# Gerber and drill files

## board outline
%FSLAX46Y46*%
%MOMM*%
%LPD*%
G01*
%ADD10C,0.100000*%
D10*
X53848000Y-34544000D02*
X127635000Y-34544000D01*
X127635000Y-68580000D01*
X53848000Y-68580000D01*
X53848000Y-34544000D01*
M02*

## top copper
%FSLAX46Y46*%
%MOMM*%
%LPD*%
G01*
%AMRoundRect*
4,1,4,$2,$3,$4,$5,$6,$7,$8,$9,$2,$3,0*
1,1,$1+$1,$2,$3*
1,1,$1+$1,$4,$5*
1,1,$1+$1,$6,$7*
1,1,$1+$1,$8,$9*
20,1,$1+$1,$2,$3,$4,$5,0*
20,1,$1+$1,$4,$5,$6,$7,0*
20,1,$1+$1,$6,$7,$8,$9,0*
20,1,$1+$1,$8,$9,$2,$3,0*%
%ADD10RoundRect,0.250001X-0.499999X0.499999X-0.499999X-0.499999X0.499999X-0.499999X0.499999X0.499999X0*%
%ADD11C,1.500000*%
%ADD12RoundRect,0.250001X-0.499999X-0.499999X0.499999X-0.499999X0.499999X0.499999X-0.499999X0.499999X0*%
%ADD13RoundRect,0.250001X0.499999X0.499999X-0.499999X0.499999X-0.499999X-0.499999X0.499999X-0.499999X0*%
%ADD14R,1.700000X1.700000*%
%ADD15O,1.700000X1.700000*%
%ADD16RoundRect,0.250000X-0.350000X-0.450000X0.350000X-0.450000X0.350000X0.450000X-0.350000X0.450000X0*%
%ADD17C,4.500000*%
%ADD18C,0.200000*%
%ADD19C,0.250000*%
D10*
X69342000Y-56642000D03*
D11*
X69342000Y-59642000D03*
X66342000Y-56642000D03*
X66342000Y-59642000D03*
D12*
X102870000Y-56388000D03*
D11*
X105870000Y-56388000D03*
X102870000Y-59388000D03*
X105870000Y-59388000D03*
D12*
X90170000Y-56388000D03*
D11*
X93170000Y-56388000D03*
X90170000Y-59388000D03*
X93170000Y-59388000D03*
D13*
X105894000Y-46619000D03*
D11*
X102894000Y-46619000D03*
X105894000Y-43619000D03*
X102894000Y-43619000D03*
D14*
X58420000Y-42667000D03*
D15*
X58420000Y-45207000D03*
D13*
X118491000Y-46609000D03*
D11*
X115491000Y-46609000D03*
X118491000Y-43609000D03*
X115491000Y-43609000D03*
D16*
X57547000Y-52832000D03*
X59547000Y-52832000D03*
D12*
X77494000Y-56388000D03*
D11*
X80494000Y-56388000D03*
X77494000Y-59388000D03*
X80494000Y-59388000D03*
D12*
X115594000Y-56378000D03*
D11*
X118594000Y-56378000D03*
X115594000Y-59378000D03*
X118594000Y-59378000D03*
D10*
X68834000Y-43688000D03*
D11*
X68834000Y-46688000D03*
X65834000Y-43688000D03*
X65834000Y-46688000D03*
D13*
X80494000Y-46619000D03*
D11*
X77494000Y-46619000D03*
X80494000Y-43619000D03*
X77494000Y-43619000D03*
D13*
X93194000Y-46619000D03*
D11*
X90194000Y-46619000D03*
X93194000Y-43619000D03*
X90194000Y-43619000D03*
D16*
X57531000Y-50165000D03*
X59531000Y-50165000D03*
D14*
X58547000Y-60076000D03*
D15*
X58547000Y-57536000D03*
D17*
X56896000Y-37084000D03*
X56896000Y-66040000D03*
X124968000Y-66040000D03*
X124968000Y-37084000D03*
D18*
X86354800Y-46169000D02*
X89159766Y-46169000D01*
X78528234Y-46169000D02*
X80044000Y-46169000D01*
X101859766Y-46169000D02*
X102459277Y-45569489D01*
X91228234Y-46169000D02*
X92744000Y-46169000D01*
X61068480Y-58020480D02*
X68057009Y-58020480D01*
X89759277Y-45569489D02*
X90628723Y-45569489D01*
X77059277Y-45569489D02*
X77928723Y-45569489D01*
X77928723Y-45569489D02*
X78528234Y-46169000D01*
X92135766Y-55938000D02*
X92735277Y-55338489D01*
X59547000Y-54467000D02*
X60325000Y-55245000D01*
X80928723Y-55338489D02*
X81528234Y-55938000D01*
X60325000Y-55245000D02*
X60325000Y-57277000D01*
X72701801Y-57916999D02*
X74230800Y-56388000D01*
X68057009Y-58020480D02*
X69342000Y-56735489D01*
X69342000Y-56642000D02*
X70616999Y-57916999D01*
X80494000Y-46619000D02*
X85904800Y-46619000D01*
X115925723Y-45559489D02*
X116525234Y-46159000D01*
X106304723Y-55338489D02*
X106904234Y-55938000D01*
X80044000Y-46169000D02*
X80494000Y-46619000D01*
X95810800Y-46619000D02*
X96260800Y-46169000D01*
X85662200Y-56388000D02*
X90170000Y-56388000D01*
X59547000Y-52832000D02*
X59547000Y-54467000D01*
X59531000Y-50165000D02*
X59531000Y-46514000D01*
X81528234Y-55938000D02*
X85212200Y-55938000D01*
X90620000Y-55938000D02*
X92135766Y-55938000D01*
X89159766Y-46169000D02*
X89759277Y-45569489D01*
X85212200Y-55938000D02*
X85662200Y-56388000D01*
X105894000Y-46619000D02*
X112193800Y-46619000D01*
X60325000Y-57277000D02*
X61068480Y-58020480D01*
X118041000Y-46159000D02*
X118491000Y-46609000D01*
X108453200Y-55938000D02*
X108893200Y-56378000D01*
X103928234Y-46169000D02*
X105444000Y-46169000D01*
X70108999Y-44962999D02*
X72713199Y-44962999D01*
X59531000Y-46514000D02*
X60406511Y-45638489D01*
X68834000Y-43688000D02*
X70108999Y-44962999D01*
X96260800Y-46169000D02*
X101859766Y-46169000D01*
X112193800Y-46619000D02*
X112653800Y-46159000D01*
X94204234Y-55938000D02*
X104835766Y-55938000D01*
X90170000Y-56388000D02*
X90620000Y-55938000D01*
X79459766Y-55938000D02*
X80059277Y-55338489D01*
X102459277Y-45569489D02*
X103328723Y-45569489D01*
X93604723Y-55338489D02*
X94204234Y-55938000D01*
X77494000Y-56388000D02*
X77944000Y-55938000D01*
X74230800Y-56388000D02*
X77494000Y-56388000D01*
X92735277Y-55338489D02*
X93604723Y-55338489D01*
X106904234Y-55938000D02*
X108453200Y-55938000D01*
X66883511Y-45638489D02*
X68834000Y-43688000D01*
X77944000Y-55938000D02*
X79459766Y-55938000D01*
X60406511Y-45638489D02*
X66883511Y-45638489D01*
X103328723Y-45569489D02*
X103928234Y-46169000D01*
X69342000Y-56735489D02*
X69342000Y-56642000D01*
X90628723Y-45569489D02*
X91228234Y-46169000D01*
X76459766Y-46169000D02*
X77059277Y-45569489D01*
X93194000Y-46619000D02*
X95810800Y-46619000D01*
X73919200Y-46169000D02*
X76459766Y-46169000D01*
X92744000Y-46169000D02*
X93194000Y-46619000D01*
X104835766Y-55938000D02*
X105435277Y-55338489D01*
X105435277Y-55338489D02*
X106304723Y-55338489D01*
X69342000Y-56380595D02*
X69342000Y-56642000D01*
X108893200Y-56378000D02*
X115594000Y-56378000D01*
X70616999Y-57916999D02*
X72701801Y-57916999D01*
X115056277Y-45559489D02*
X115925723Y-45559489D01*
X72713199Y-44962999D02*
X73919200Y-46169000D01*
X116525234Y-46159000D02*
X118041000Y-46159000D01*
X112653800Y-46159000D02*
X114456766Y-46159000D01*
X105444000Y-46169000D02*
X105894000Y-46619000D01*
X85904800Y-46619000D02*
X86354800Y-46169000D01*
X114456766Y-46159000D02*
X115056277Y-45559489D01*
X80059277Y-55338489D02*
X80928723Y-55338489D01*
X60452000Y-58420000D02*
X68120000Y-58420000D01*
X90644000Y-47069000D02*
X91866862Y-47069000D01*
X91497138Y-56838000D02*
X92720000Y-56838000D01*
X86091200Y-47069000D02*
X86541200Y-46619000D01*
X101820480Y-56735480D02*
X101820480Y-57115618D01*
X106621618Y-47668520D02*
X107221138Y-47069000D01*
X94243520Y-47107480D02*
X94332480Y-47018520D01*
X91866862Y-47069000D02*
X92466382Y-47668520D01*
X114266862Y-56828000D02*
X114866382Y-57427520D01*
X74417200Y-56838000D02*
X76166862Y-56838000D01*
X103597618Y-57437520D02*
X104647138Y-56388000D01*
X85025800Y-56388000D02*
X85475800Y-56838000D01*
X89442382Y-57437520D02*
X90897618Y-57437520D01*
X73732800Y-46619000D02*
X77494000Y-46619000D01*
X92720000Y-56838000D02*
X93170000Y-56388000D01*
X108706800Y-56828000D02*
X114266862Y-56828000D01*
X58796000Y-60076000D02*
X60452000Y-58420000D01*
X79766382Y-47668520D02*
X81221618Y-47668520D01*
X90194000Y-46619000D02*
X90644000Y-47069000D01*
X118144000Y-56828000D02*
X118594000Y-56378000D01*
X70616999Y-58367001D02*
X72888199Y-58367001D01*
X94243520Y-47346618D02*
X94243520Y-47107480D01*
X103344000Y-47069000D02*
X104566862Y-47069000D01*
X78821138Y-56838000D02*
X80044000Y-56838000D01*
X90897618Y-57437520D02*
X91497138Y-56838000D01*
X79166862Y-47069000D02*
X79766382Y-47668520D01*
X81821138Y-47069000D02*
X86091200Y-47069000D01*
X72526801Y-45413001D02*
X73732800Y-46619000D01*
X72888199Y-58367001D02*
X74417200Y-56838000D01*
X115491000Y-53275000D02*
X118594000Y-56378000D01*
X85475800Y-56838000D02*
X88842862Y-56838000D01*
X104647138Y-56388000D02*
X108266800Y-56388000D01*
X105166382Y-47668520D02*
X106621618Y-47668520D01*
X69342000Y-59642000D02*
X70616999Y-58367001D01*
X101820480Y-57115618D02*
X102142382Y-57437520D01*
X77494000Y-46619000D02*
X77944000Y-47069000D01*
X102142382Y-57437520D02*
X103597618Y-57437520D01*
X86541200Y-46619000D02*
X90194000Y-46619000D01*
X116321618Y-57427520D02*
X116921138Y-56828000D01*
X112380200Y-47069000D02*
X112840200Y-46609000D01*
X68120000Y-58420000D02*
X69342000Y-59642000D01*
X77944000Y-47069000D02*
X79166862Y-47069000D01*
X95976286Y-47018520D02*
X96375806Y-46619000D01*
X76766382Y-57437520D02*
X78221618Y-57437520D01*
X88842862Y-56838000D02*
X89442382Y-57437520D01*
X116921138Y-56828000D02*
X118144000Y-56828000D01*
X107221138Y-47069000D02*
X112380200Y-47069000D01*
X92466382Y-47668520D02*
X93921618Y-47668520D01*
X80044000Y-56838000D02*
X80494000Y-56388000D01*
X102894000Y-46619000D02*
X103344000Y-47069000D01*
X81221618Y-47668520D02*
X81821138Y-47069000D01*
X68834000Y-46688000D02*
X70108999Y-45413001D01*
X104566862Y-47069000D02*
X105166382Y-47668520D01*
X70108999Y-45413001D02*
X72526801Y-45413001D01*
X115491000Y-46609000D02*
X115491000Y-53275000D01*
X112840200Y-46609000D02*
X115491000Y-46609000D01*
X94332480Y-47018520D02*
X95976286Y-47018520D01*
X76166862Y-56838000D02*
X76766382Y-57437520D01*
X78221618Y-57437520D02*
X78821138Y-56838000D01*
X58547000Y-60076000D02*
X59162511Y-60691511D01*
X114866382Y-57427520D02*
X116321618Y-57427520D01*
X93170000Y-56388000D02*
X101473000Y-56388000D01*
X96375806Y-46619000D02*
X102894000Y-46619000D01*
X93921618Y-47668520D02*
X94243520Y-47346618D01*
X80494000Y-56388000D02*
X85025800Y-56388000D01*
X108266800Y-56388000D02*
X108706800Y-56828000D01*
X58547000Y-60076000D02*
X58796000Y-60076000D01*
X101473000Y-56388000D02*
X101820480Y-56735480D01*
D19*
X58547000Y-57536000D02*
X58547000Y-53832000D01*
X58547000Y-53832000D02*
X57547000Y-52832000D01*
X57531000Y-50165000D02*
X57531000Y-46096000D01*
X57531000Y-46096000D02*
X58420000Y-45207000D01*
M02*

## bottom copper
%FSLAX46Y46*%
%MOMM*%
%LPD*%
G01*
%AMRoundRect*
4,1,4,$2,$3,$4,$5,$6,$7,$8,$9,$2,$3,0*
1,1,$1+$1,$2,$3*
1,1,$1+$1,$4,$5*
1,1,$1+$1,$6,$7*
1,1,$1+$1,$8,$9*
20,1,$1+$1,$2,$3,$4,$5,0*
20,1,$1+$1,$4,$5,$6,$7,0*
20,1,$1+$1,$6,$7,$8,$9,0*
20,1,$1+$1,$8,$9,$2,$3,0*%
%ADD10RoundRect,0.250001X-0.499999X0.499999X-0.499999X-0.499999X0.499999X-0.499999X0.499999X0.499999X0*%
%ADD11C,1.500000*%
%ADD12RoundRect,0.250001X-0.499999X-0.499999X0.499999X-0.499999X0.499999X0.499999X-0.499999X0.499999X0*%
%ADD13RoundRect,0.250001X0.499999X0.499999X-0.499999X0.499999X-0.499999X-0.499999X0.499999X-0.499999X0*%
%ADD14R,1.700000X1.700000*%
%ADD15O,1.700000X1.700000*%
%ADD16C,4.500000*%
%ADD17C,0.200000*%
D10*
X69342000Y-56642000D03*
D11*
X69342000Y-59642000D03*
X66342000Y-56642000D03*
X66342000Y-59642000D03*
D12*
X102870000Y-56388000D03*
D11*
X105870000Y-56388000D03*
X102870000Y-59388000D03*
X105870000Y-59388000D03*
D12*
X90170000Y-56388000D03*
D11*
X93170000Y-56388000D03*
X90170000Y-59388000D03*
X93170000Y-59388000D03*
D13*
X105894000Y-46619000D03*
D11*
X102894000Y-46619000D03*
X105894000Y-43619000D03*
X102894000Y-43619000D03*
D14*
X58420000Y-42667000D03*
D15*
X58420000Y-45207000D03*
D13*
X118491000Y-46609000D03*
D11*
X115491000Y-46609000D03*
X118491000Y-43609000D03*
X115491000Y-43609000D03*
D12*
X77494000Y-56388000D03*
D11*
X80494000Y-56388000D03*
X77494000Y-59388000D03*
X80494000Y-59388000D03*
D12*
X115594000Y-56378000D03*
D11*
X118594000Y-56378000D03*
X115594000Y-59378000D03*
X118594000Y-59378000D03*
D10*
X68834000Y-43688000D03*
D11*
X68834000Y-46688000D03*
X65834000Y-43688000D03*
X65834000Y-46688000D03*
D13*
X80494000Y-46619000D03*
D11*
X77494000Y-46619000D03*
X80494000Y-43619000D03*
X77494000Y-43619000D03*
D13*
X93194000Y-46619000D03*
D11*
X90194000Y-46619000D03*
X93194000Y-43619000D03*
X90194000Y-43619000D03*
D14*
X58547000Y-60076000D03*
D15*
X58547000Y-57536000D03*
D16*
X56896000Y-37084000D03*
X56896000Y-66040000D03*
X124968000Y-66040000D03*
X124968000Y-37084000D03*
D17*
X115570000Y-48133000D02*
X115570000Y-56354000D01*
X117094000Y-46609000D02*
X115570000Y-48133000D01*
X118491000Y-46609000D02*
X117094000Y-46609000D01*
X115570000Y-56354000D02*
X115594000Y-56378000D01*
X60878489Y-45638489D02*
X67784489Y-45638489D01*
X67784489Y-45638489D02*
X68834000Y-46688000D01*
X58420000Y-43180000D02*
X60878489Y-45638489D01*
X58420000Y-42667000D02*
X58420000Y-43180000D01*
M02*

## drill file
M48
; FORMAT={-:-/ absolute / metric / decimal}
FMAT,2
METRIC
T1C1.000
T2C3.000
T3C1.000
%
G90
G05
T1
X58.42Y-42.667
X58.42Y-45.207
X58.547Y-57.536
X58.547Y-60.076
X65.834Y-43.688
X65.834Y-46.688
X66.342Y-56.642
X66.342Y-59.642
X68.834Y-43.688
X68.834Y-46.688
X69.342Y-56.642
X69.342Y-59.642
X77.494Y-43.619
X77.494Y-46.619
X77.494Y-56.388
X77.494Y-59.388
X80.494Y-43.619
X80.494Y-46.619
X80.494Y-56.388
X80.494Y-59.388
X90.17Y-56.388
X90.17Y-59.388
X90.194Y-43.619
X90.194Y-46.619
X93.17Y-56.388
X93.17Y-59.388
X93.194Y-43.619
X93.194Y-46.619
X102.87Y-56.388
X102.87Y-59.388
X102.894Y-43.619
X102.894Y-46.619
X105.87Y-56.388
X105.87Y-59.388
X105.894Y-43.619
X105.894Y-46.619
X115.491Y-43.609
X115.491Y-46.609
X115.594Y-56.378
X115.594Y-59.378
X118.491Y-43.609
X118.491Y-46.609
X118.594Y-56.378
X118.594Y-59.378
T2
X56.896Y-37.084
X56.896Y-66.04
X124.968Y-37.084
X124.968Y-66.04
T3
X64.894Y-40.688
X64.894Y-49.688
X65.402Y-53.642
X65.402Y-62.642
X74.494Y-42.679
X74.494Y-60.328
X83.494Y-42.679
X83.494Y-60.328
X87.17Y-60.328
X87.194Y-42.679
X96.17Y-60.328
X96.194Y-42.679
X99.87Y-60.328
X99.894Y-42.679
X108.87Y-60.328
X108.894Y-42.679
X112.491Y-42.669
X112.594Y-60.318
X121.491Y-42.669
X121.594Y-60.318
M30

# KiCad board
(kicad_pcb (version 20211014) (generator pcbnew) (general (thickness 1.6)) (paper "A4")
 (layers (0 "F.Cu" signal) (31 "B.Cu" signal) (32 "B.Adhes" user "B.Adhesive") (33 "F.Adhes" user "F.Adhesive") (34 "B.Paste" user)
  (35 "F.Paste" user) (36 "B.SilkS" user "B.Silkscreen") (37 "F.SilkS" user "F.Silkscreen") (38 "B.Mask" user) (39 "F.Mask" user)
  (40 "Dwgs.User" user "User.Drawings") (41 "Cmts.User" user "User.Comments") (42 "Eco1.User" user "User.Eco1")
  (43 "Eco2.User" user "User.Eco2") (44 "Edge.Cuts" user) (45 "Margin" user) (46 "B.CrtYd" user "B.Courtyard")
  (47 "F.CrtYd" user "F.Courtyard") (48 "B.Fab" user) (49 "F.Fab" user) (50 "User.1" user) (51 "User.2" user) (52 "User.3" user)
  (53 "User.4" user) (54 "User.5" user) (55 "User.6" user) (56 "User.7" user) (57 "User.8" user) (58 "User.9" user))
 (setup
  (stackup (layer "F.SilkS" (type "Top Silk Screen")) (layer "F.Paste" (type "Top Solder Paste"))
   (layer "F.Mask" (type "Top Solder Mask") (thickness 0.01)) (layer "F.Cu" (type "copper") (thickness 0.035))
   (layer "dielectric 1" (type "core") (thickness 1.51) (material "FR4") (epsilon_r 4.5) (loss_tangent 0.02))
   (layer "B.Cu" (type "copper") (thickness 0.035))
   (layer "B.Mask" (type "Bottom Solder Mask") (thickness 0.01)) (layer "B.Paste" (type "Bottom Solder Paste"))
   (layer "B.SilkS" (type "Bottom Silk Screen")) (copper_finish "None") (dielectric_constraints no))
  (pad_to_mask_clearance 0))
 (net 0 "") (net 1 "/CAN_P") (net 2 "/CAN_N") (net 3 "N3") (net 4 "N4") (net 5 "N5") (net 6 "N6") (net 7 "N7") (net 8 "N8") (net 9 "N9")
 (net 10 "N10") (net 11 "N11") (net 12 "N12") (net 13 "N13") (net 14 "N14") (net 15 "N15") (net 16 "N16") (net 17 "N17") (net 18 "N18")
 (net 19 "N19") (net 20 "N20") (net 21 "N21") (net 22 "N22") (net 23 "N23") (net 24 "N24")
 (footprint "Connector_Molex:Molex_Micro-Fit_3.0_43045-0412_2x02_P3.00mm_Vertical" (layer "F.Cu") (at 69.342 56.642 -90)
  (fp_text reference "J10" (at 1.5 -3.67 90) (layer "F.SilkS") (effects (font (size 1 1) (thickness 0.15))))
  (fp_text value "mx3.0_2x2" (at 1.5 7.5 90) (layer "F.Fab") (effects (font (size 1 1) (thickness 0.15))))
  (pad "" np_thru_hole circle locked (at -3 3.94 270) (size 1 1) (drill 1) (layers *.Cu *.Mask))
  (pad "" np_thru_hole circle locked (at 6 3.94 270) (size 1 1) (drill 1) (layers *.Cu *.Mask))
  (pad "1" thru_hole roundrect locked (at 0 0 270) (size 1.5 1.5) (drill 1) (layers *.Cu *.Mask) (roundrect_rratio 0.166667)
   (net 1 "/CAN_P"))
  (pad "2" thru_hole circle locked (at 3 0 270) (size 1.5 1.5) (drill 1) (layers *.Cu *.Mask) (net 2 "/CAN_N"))
  (pad "3" thru_hole circle locked (at 0 3 270) (size 1.5 1.5) (drill 1) (layers *.Cu *.Mask) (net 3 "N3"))
  (pad "4" thru_hole circle locked (at 3 3 270) (size 1.5 1.5) (drill 1) (layers *.Cu *.Mask) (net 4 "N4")))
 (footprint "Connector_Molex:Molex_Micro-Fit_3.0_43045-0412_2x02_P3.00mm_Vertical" (layer "F.Cu") (at 102.87 56.388)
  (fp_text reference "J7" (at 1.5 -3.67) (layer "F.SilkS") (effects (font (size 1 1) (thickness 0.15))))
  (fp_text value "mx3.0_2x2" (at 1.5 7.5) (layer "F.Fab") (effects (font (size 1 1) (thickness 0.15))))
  (pad "" np_thru_hole circle locked (at 6 3.94) (size 1 1) (drill 1) (layers *.Cu *.Mask))
  (pad "" np_thru_hole circle locked (at -3 3.94) (size 1 1) (drill 1) (layers *.Cu *.Mask))
  (pad "1" thru_hole roundrect locked (at 0 0) (size 1.5 1.5) (drill 1) (layers *.Cu *.Mask) (roundrect_rratio 0.166667) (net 1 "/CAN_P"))
  (pad "2" thru_hole circle locked (at 3 0) (size 1.5 1.5) (drill 1) (layers *.Cu *.Mask) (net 2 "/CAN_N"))
  (pad "3" thru_hole circle locked (at 0 3) (size 1.5 1.5) (drill 1) (layers *.Cu *.Mask) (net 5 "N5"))
  (pad "4" thru_hole circle locked (at 3 3) (size 1.5 1.5) (drill 1) (layers *.Cu *.Mask) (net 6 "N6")))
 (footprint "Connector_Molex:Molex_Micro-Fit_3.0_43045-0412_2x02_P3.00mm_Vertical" (layer "F.Cu") (at 90.17 56.388)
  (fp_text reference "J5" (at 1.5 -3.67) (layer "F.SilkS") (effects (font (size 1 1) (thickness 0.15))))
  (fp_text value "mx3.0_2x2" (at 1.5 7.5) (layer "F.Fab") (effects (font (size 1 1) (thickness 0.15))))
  (pad "" np_thru_hole circle locked (at -3 3.94) (size 1 1) (drill 1) (layers *.Cu *.Mask))
  (pad "" np_thru_hole circle locked (at 6 3.94) (size 1 1) (drill 1) (layers *.Cu *.Mask))
  (pad "1" thru_hole roundrect locked (at 0 0) (size 1.5 1.5) (drill 1) (layers *.Cu *.Mask) (roundrect_rratio 0.166667) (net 1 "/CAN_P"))
  (pad "2" thru_hole circle locked (at 3 0) (size 1.5 1.5) (drill 1) (layers *.Cu *.Mask) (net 2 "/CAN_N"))
  (pad "3" thru_hole circle locked (at 0 3) (size 1.5 1.5) (drill 1) (layers *.Cu *.Mask) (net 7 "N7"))
  (pad "4" thru_hole circle locked (at 3 3) (size 1.5 1.5) (drill 1) (layers *.Cu *.Mask) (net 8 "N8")))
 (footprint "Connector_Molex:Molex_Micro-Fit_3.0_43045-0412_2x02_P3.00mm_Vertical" (layer "F.Cu") (at 105.894 46.619 180)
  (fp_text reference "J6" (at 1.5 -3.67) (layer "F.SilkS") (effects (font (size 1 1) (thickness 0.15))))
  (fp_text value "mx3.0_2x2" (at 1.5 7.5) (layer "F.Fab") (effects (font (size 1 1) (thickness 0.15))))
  (pad "" np_thru_hole circle locked (at 6 3.94 180) (size 1 1) (drill 1) (layers *.Cu *.Mask))
  (pad "" np_thru_hole circle locked (at -3 3.94 180) (size 1 1) (drill 1) (layers *.Cu *.Mask))
  (pad "1" thru_hole roundrect locked (at 0 0 180) (size 1.5 1.5) (drill 1) (layers *.Cu *.Mask) (roundrect_rratio 0.166667)
   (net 1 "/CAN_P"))
  (pad "2" thru_hole circle locked (at 3 0 180) (size 1.5 1.5) (drill 1) (layers *.Cu *.Mask) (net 2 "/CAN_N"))
  (pad "3" thru_hole circle locked (at 0 3 180) (size 1.5 1.5) (drill 1) (layers *.Cu *.Mask) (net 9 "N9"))
  (pad "4" thru_hole circle locked (at 3 3 180) (size 1.5 1.5) (drill 1) (layers *.Cu *.Mask) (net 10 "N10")))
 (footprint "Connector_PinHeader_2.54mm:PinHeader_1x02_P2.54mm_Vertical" (layer "F.Cu") (at 58.42 42.667)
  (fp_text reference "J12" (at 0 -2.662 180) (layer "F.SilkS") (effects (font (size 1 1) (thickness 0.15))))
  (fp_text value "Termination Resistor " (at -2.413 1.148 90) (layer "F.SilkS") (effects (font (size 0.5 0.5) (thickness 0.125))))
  (pad "1" thru_hole rect locked (at 0 0) (size 1.7 1.7) (drill 1) (layers *.Cu *.Mask) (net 2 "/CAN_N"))
  (pad "2" thru_hole oval locked (at 0 2.54) (size 1.7 1.7) (drill 1) (layers *.Cu *.Mask) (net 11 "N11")))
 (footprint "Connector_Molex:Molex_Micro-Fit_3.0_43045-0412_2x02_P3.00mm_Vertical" (layer "F.Cu") (at 118.491 46.609 180)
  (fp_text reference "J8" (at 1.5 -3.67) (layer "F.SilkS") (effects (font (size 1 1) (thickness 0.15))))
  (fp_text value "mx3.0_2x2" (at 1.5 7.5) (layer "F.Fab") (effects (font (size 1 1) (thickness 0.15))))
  (pad "" np_thru_hole circle locked (at 6 3.94 180) (size 1 1) (drill 1) (layers *.Cu *.Mask))
  (pad "" np_thru_hole circle locked (at -3 3.94 180) (size 1 1) (drill 1) (layers *.Cu *.Mask))
  (pad "1" thru_hole roundrect locked (at 0 0 180) (size 1.5 1.5) (drill 1) (layers *.Cu *.Mask) (roundrect_rratio 0.166667)
   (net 1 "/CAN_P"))
  (pad "2" thru_hole circle locked (at 3 0 180) (size 1.5 1.5) (drill 1) (layers *.Cu *.Mask) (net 2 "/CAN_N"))
  (pad "3" thru_hole circle locked (at 0 3 180) (size 1.5 1.5) (drill 1) (layers *.Cu *.Mask) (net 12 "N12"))
  (pad "4" thru_hole circle locked (at 3 3 180) (size 1.5 1.5) (drill 1) (layers *.Cu *.Mask) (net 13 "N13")))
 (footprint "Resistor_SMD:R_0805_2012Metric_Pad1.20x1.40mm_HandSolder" (layer "F.Cu") (at 58.547 52.832)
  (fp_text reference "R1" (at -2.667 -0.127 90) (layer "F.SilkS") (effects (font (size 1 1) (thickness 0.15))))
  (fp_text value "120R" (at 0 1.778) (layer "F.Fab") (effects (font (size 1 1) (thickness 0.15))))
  (pad "1" smd roundrect locked (at -1 0) (size 1.2 1.4) (layers "F.Cu" "F.Paste" "F.Mask") (roundrect_rratio 0.208333) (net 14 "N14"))
  (pad "2" smd roundrect locked (at 1 0) (size 1.2 1.4) (layers "F.Cu" "F.Paste" "F.Mask") (roundrect_rratio 0.208333) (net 1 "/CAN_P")))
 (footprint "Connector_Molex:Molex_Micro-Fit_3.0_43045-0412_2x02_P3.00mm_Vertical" (layer "F.Cu") (at 77.494 56.388)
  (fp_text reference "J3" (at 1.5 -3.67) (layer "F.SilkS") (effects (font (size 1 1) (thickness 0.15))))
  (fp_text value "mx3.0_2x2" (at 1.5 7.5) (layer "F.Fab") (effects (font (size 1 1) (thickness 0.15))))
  (pad "" np_thru_hole circle locked (at -3 3.94) (size 1 1) (drill 1) (layers *.Cu *.Mask))
  (pad "" np_thru_hole circle locked (at 6 3.94) (size 1 1) (drill 1) (layers *.Cu *.Mask))
  (pad "1" thru_hole roundrect locked (at 0 0) (size 1.5 1.5) (drill 1) (layers *.Cu *.Mask) (roundrect_rratio 0.166667) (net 1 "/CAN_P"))
  (pad "2" thru_hole circle locked (at 3 0) (size 1.5 1.5) (drill 1) (layers *.Cu *.Mask) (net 2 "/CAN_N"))
  (pad "3" thru_hole circle locked (at 0 3) (size 1.5 1.5) (drill 1) (layers *.Cu *.Mask) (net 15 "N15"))
  (pad "4" thru_hole circle locked (at 3 3) (size 1.5 1.5) (drill 1) (layers *.Cu *.Mask) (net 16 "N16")))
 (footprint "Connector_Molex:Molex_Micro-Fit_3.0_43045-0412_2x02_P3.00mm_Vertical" (layer "F.Cu") (at 115.594 56.378)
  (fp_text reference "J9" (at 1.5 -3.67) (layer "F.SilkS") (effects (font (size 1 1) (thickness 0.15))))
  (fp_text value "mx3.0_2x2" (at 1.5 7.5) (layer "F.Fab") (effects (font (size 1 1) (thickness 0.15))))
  (pad "" np_thru_hole circle locked (at 6 3.94) (size 1 1) (drill 1) (layers *.Cu *.Mask))
  (pad "" np_thru_hole circle locked (at -3 3.94) (size 1 1) (drill 1) (layers *.Cu *.Mask))
  (pad "1" thru_hole roundrect locked (at 0 0) (size 1.5 1.5) (drill 1) (layers *.Cu *.Mask) (roundrect_rratio 0.166667) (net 1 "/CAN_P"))
  (pad "2" thru_hole circle locked (at 3 0) (size 1.5 1.5) (drill 1) (layers *.Cu *.Mask) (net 2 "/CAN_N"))
  (pad "3" thru_hole circle locked (at 0 3) (size 1.5 1.5) (drill 1) (layers *.Cu *.Mask) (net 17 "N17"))
  (pad "4" thru_hole circle locked (at 3 3) (size 1.5 1.5) (drill 1) (layers *.Cu *.Mask) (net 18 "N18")))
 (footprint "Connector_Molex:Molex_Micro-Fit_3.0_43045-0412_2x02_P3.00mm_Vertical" (layer "F.Cu") (at 68.834 43.688 -90)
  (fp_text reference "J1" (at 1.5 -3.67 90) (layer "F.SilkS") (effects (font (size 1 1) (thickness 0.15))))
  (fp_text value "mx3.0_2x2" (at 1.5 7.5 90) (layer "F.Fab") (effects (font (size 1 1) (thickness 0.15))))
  (pad "" np_thru_hole circle locked (at -3 3.94 270) (size 1 1) (drill 1) (layers *.Cu *.Mask))
  (pad "" np_thru_hole circle locked (at 6 3.94 270) (size 1 1) (drill 1) (layers *.Cu *.Mask))
  (pad "1" thru_hole roundrect locked (at 0 0 270) (size 1.5 1.5) (drill 1) (layers *.Cu *.Mask) (roundrect_rratio 0.166667)
   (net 1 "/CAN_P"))
  (pad "2" thru_hole circle locked (at 3 0 270) (size 1.5 1.5) (drill 1) (layers *.Cu *.Mask) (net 2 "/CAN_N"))
  (pad "3" thru_hole circle locked (at 0 3 270) (size 1.5 1.5) (drill 1) (layers *.Cu *.Mask) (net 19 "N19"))
  (pad "4" thru_hole circle locked (at 3 3 270) (size 1.5 1.5) (drill 1) (layers *.Cu *.Mask) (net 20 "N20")))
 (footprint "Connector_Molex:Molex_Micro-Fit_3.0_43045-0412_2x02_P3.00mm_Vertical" (layer "F.Cu") (at 80.494 46.619 180)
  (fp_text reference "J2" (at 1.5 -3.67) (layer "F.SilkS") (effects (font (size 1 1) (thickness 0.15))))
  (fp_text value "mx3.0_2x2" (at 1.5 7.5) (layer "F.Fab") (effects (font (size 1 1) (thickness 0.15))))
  (pad "" np_thru_hole circle locked (at -3 3.94 180) (size 1 1) (drill 1) (layers *.Cu *.Mask))
  (pad "" np_thru_hole circle locked (at 6 3.94 180) (size 1 1) (drill 1) (layers *.Cu *.Mask))
  (pad "1" thru_hole roundrect locked (at 0 0 180) (size 1.5 1.5) (drill 1) (layers *.Cu *.Mask) (roundrect_rratio 0.166667)
   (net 1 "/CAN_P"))
  (pad "2" thru_hole circle locked (at 3 0 180) (size 1.5 1.5) (drill 1) (layers *.Cu *.Mask) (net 2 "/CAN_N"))
  (pad "3" thru_hole circle locked (at 0 3 180) (size 1.5 1.5) (drill 1) (layers *.Cu *.Mask) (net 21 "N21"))
  (pad "4" thru_hole circle locked (at 3 3 180) (size 1.5 1.5) (drill 1) (layers *.Cu *.Mask) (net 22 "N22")))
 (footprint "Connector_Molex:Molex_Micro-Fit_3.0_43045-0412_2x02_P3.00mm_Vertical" (layer "F.Cu") (at 93.194 46.619 180)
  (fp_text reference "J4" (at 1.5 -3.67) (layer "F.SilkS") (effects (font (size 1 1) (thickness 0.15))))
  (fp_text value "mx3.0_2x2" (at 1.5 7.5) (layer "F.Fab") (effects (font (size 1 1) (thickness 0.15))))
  (pad "" np_thru_hole circle locked (at -3 3.94 180) (size 1 1) (drill 1) (layers *.Cu *.Mask))
  (pad "" np_thru_hole circle locked (at 6 3.94 180) (size 1 1) (drill 1) (layers *.Cu *.Mask))
  (pad "1" thru_hole roundrect locked (at 0 0 180) (size 1.5 1.5) (drill 1) (layers *.Cu *.Mask) (roundrect_rratio 0.166667)
   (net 1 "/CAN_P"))
  (pad "2" thru_hole circle locked (at 3 0 180) (size 1.5 1.5) (drill 1) (layers *.Cu *.Mask) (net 2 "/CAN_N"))
  (pad "3" thru_hole circle locked (at 0 3 180) (size 1.5 1.5) (drill 1) (layers *.Cu *.Mask) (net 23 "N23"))
  (pad "4" thru_hole circle locked (at 3 3 180) (size 1.5 1.5) (drill 1) (layers *.Cu *.Mask) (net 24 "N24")))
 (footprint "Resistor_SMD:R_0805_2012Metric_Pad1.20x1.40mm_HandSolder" (layer "F.Cu") (at 58.531 50.165)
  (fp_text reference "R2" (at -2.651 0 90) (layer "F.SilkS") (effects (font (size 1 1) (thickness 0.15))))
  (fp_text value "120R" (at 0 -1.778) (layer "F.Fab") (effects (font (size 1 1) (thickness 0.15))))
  (pad "1" smd roundrect locked (at -1 0) (size 1.2 1.4) (layers "F.Cu" "F.Paste" "F.Mask") (roundrect_rratio 0.208333) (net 11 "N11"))
  (pad "2" smd roundrect locked (at 1 0) (size 1.2 1.4) (layers "F.Cu" "F.Paste" "F.Mask") (roundrect_rratio 0.208333) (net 1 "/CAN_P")))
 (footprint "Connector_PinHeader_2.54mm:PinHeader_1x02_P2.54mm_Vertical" (layer "F.Cu") (at 58.547 60.076 180)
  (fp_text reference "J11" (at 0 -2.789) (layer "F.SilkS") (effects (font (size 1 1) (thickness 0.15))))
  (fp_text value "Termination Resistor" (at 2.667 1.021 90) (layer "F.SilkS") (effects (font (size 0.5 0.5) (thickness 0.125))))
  (pad "1" thru_hole rect locked (at 0 0 180) (size 1.7 1.7) (drill 1) (layers *.Cu *.Mask) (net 2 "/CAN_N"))
  (pad "2" thru_hole oval locked (at 0 2.54 180) (size 1.7 1.7) (drill 1) (layers *.Cu *.Mask) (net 14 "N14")))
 (gr_rect (start 127.635 34.544) (end 53.848 68.58) (layer "Edge.Cuts") (width 0.1) (fill none))
 (via (at 56.896 37.084) (size 4.5) (drill 3) (layers "F.Cu" "B.Cu") (free) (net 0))
 (via (at 56.896 66.04) (size 4.5) (drill 3) (layers "F.Cu" "B.Cu") (free) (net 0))
 (via (at 124.968 66.04) (size 4.5) (drill 3) (layers "F.Cu" "B.Cu") (free) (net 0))
 (via (at 124.968 37.084) (size 4.5) (drill 3) (layers "F.Cu" "B.Cu") (free) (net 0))
 (segment (start 86.3548 46.169) (end 89.159766 46.169) (width 0.2) (layer "F.Cu") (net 1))
 (segment (start 78.528234 46.169) (end 80.044 46.169) (width 0.2) (layer "F.Cu") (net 1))
 (segment (start 101.859766 46.169) (end 102.459277 45.569489) (width 0.2) (layer "F.Cu") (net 1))
 (segment (start 91.228234 46.169) (end 92.744 46.169) (width 0.2) (layer "F.Cu") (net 1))
 (segment (start 61.06848 58.02048) (end 68.057009 58.02048) (width 0.2) (layer "F.Cu") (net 1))
 (segment (start 89.759277 45.569489) (end 90.628723 45.569489) (width 0.2) (layer "F.Cu") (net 1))
 (segment (start 77.059277 45.569489) (end 77.928723 45.569489) (width 0.2) (layer "F.Cu") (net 1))
 (segment (start 77.928723 45.569489) (end 78.528234 46.169) (width 0.2) (layer "F.Cu") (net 1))
 (segment (start 92.135766 55.938) (end 92.735277 55.338489) (width 0.2) (layer "F.Cu") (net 1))
 (segment (start 59.547 54.467) (end 60.325 55.245) (width 0.2) (layer "F.Cu") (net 1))
 (segment (start 80.928723 55.338489) (end 81.528234 55.938) (width 0.2) (layer "F.Cu") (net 1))
 (segment (start 60.325 55.245) (end 60.325 57.277) (width 0.2) (layer "F.Cu") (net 1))
 (segment (start 72.701801 57.916999) (end 74.2308 56.388) (width 0.2) (layer "F.Cu") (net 1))
 (segment (start 68.057009 58.02048) (end 69.342 56.735489) (width 0.2) (layer "F.Cu") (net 1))
 (segment (start 69.342 56.642) (end 70.616999 57.916999) (width 0.2) (layer "F.Cu") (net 1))
 (segment (start 80.494 46.619) (end 85.9048 46.619) (width 0.2) (layer "F.Cu") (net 1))
 (segment (start 115.925723 45.559489) (end 116.525234 46.159) (width 0.2) (layer "F.Cu") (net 1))
 (segment (start 106.304723 55.338489) (end 106.904234 55.938) (width 0.2) (layer "F.Cu") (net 1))
 (segment (start 80.044 46.169) (end 80.494 46.619) (width 0.2) (layer "F.Cu") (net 1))
 (segment (start 95.8108 46.619) (end 96.2608 46.169) (width 0.2) (layer "F.Cu") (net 1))
 (segment (start 85.6622 56.388) (end 90.17 56.388) (width 0.2) (layer "F.Cu") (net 1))
 (segment (start 59.547 52.832) (end 59.547 54.467) (width 0.2) (layer "F.Cu") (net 1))
 (segment (start 59.531 50.165) (end 59.531 46.514) (width 0.2) (layer "F.Cu") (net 1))
 (segment (start 81.528234 55.938) (end 85.2122 55.938) (width 0.2) (layer "F.Cu") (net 1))
 (segment (start 90.62 55.938) (end 92.135766 55.938) (width 0.2) (layer "F.Cu") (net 1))
 (segment (start 89.159766 46.169) (end 89.759277 45.569489) (width 0.2) (layer "F.Cu") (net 1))
 (segment (start 85.2122 55.938) (end 85.6622 56.388) (width 0.2) (layer "F.Cu") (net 1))
 (segment (start 105.894 46.619) (end 112.1938 46.619) (width 0.2) (layer "F.Cu") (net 1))
 (segment (start 60.325 57.277) (end 61.06848 58.02048) (width 0.2) (layer "F.Cu") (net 1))
 (segment (start 118.041 46.159) (end 118.491 46.609) (width 0.2) (layer "F.Cu") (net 1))
 (segment (start 108.4532 55.938) (end 108.8932 56.378) (width 0.2) (layer "F.Cu") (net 1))
 (segment (start 103.928234 46.169) (end 105.444 46.169) (width 0.2) (layer "F.Cu") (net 1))
 (segment (start 70.108999 44.962999) (end 72.713199 44.962999) (width 0.2) (layer "F.Cu") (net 1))
 (segment (start 59.531 46.514) (end 60.406511 45.638489) (width 0.2) (layer "F.Cu") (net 1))
 (segment (start 68.834 43.688) (end 70.108999 44.962999) (width 0.2) (layer "F.Cu") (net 1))
 (segment (start 96.2608 46.169) (end 101.859766 46.169) (width 0.2) (layer "F.Cu") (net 1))
 (segment (start 112.1938 46.619) (end 112.6538 46.159) (width 0.2) (layer "F.Cu") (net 1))
 (segment (start 94.204234 55.938) (end 104.835766 55.938) (width 0.2) (layer "F.Cu") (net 1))
 (segment (start 90.17 56.388) (end 90.62 55.938) (width 0.2) (layer "F.Cu") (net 1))
 (segment (start 79.459766 55.938) (end 80.059277 55.338489) (width 0.2) (layer "F.Cu") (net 1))
 (segment (start 102.459277 45.569489) (end 103.328723 45.569489) (width 0.2) (layer "F.Cu") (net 1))
 (segment (start 93.604723 55.338489) (end 94.204234 55.938) (width 0.2) (layer "F.Cu") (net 1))
 (segment (start 77.494 56.388) (end 77.944 55.938) (width 0.2) (layer "F.Cu") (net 1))
 (segment (start 74.2308 56.388) (end 77.494 56.388) (width 0.2) (layer "F.Cu") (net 1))
 (segment (start 92.735277 55.338489) (end 93.604723 55.338489) (width 0.2) (layer "F.Cu") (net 1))
 (segment (start 106.904234 55.938) (end 108.4532 55.938) (width 0.2) (layer "F.Cu") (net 1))
 (segment (start 66.883511 45.638489) (end 68.834 43.688) (width 0.2) (layer "F.Cu") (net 1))
 (segment (start 77.944 55.938) (end 79.459766 55.938) (width 0.2) (layer "F.Cu") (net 1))
 (segment (start 60.406511 45.638489) (end 66.883511 45.638489) (width 0.2) (layer "F.Cu") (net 1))
 (segment (start 103.328723 45.569489) (end 103.928234 46.169) (width 0.2) (layer "F.Cu") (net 1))
 (segment (start 69.342 56.735489) (end 69.342 56.642) (width 0.2) (layer "F.Cu") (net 1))
 (segment (start 90.628723 45.569489) (end 91.228234 46.169) (width 0.2) (layer "F.Cu") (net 1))
 (segment (start 76.459766 46.169) (end 77.059277 45.569489) (width 0.2) (layer "F.Cu") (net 1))
 (segment (start 93.194 46.619) (end 95.8108 46.619) (width 0.2) (layer "F.Cu") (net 1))
 (segment (start 73.9192 46.169) (end 76.459766 46.169) (width 0.2) (layer "F.Cu") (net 1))
 (segment (start 92.744 46.169) (end 93.194 46.619) (width 0.2) (layer "F.Cu") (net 1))
 (segment (start 104.835766 55.938) (end 105.435277 55.338489) (width 0.2) (layer "F.Cu") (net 1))
 (segment (start 105.435277 55.338489) (end 106.304723 55.338489) (width 0.2) (layer "F.Cu") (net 1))
 (segment (start 69.342 56.380595) (end 69.342 56.642) (width 0.2) (layer "F.Cu") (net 1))
 (segment (start 108.8932 56.378) (end 115.594 56.378) (width 0.2) (layer "F.Cu") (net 1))
 (segment (start 70.616999 57.916999) (end 72.701801 57.916999) (width 0.2) (layer "F.Cu") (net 1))
 (segment (start 115.056277 45.559489) (end 115.925723 45.559489) (width 0.2) (layer "F.Cu") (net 1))
 (segment (start 72.713199 44.962999) (end 73.9192 46.169) (width 0.2) (layer "F.Cu") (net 1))
 (segment (start 116.525234 46.159) (end 118.041 46.159) (width 0.2) (layer "F.Cu") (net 1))
 (segment (start 112.6538 46.159) (end 114.456766 46.159) (width 0.2) (layer "F.Cu") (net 1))
 (segment (start 105.444 46.169) (end 105.894 46.619) (width 0.2) (layer "F.Cu") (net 1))
 (segment (start 85.9048 46.619) (end 86.3548 46.169) (width 0.2) (layer "F.Cu") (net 1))
 (segment (start 114.456766 46.159) (end 115.056277 45.559489) (width 0.2) (layer "F.Cu") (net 1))
 (segment (start 80.059277 55.338489) (end 80.928723 55.338489) (width 0.2) (layer "F.Cu") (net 1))
 (segment (start 115.57 48.133) (end 115.57 56.354) (width 0.2) (layer "B.Cu") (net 1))
 (segment (start 117.094 46.609) (end 115.57 48.133) (width 0.2) (layer "B.Cu") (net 1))
 (segment (start 118.491 46.609) (end 117.094 46.609) (width 0.2) (layer "B.Cu") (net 1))
 (segment (start 115.57 56.354) (end 115.594 56.378) (width 0.2) (layer "B.Cu") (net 1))
 (segment (start 60.452 58.42) (end 68.12 58.42) (width 0.2) (layer "F.Cu") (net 2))
 (segment (start 90.644 47.069) (end 91.866862 47.069) (width 0.2) (layer "F.Cu") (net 2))
 (segment (start 91.497138 56.838) (end 92.72 56.838) (width 0.2) (layer "F.Cu") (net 2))
 (segment (start 86.0912 47.069) (end 86.5412 46.619) (width 0.2) (layer "F.Cu") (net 2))
 (segment (start 101.82048 56.73548) (end 101.82048 57.115618) (width 0.2) (layer "F.Cu") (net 2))
 (segment (start 106.621618 47.66852) (end 107.221138 47.069) (width 0.2) (layer "F.Cu") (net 2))
 (segment (start 94.24352 47.10748) (end 94.33248 47.01852) (width 0.2) (layer "F.Cu") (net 2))
 (segment (start 91.866862 47.069) (end 92.466382 47.66852) (width 0.2) (layer "F.Cu") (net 2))
 (segment (start 114.266862 56.828) (end 114.866382 57.42752) (width 0.2) (layer "F.Cu") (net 2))
 (segment (start 74.4172 56.838) (end 76.166862 56.838) (width 0.2) (layer "F.Cu") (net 2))
 (segment (start 103.597618 57.43752) (end 104.647138 56.388) (width 0.2) (layer "F.Cu") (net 2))
 (segment (start 85.0258 56.388) (end 85.4758 56.838) (width 0.2) (layer "F.Cu") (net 2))
 (segment (start 89.442382 57.43752) (end 90.897618 57.43752) (width 0.2) (layer "F.Cu") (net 2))
 (segment (start 73.7328 46.619) (end 77.494 46.619) (width 0.2) (layer "F.Cu") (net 2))
 (segment (start 92.72 56.838) (end 93.17 56.388) (width 0.2) (layer "F.Cu") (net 2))
 (segment (start 108.7068 56.828) (end 114.266862 56.828) (width 0.2) (layer "F.Cu") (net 2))
 (segment (start 58.796 60.076) (end 60.452 58.42) (width 0.2) (layer "F.Cu") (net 2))
 (segment (start 79.766382 47.66852) (end 81.221618 47.66852) (width 0.2) (layer "F.Cu") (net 2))
 (segment (start 90.194 46.619) (end 90.644 47.069) (width 0.2) (layer "F.Cu") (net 2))
 (segment (start 118.144 56.828) (end 118.594 56.378) (width 0.2) (layer "F.Cu") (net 2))
 (segment (start 70.616999 58.367001) (end 72.888199 58.367001) (width 0.2) (layer "F.Cu") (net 2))
 (segment (start 94.24352 47.346618) (end 94.24352 47.10748) (width 0.2) (layer "F.Cu") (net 2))
 (segment (start 103.344 47.069) (end 104.566862 47.069) (width 0.2) (layer "F.Cu") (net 2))
 (segment (start 78.821138 56.838) (end 80.044 56.838) (width 0.2) (layer "F.Cu") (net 2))
 (segment (start 90.897618 57.43752) (end 91.497138 56.838) (width 0.2) (layer "F.Cu") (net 2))
 (segment (start 79.166862 47.069) (end 79.766382 47.66852) (width 0.2) (layer "F.Cu") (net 2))
 (segment (start 81.821138 47.069) (end 86.0912 47.069) (width 0.2) (layer "F.Cu") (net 2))
 (segment (start 72.526801 45.413001) (end 73.7328 46.619) (width 0.2) (layer "F.Cu") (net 2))
 (segment (start 72.888199 58.367001) (end 74.4172 56.838) (width 0.2) (layer "F.Cu") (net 2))
 (segment (start 115.491 53.275) (end 118.594 56.378) (width 0.2) (layer "F.Cu") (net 2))
 (segment (start 85.4758 56.838) (end 88.842862 56.838) (width 0.2) (layer "F.Cu") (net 2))
 (segment (start 104.647138 56.388) (end 108.2668 56.388) (width 0.2) (layer "F.Cu") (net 2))
 (segment (start 105.166382 47.66852) (end 106.621618 47.66852) (width 0.2) (layer "F.Cu") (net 2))
 (segment (start 69.342 59.642) (end 70.616999 58.367001) (width 0.2) (layer "F.Cu") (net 2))
 (segment (start 101.82048 57.115618) (end 102.142382 57.43752) (width 0.2) (layer "F.Cu") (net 2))
 (segment (start 77.494 46.619) (end 77.944 47.069) (width 0.2) (layer "F.Cu") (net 2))
 (segment (start 102.142382 57.43752) (end 103.597618 57.43752) (width 0.2) (layer "F.Cu") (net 2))
 (segment (start 86.5412 46.619) (end 90.194 46.619) (width 0.2) (layer "F.Cu") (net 2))
 (segment (start 116.321618 57.42752) (end 116.921138 56.828) (width 0.2) (layer "F.Cu") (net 2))
 (segment (start 112.3802 47.069) (end 112.8402 46.609) (width 0.2) (layer "F.Cu") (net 2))
 (segment (start 68.12 58.42) (end 69.342 59.642) (width 0.2) (layer "F.Cu") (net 2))
 (segment (start 77.944 47.069) (end 79.166862 47.069) (width 0.2) (layer "F.Cu") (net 2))
 (segment (start 95.976286 47.01852) (end 96.375806 46.619) (width 0.2) (layer "F.Cu") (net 2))
 (segment (start 76.766382 57.43752) (end 78.221618 57.43752) (width 0.2) (layer "F.Cu") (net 2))
 (segment (start 88.842862 56.838) (end 89.442382 57.43752) (width 0.2) (layer "F.Cu") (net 2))
 (segment (start 116.921138 56.828) (end 118.144 56.828) (width 0.2) (layer "F.Cu") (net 2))
 (segment (start 107.221138 47.069) (end 112.3802 47.069) (width 0.2) (layer "F.Cu") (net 2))
 (segment (start 92.466382 47.66852) (end 93.921618 47.66852) (width 0.2) (layer "F.Cu") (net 2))
 (segment (start 80.044 56.838) (end 80.494 56.388) (width 0.2) (layer "F.Cu") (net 2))
 (segment (start 102.894 46.619) (end 103.344 47.069) (width 0.2) (layer "F.Cu") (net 2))
 (segment (start 81.221618 47.66852) (end 81.821138 47.069) (width 0.2) (layer "F.Cu") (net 2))
 (segment (start 68.834 46.688) (end 70.108999 45.413001) (width 0.2) (layer "F.Cu") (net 2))
 (segment (start 104.566862 47.069) (end 105.166382 47.66852) (width 0.2) (layer "F.Cu") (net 2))
 (segment (start 70.108999 45.413001) (end 72.526801 45.413001) (width 0.2) (layer "F.Cu") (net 2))
 (segment (start 115.491 46.609) (end 115.491 53.275) (width 0.2) (layer "F.Cu") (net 2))
 (segment (start 112.8402 46.609) (end 115.491 46.609) (width 0.2) (layer "F.Cu") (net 2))
 (segment (start 94.33248 47.01852) (end 95.976286 47.01852) (width 0.2) (layer "F.Cu") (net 2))
 (segment (start 76.166862 56.838) (end 76.766382 57.43752) (width 0.2) (layer "F.Cu") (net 2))
 (segment (start 78.221618 57.43752) (end 78.821138 56.838) (width 0.2) (layer "F.Cu") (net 2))
 (segment (start 58.547 60.076) (end 59.162511 60.691511) (width 0.2) (layer "F.Cu") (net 2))
 (segment (start 114.866382 57.42752) (end 116.321618 57.42752) (width 0.2) (layer "F.Cu") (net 2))
 (segment (start 93.17 56.388) (end 101.473 56.388) (width 0.2) (layer "F.Cu") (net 2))
 (segment (start 96.375806 46.619) (end 102.894 46.619) (width 0.2) (layer "F.Cu") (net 2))
 (segment (start 93.921618 47.66852) (end 94.24352 47.346618) (width 0.2) (layer "F.Cu") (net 2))
 (segment (start 80.494 56.388) (end 85.0258 56.388) (width 0.2) (layer "F.Cu") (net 2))
 (segment (start 108.2668 56.388) (end 108.7068 56.828) (width 0.2) (layer "F.Cu") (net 2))
 (segment (start 58.547 60.076) (end 58.796 60.076) (width 0.2) (layer "F.Cu") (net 2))
 (segment (start 101.473 56.388) (end 101.82048 56.73548) (width 0.2) (layer "F.Cu") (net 2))
 (segment (start 60.878489 45.638489) (end 67.784489 45.638489) (width 0.2) (layer "B.Cu") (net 2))
 (segment (start 67.784489 45.638489) (end 68.834 46.688) (width 0.2) (layer "B.Cu") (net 2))
 (segment (start 58.42 43.18) (end 60.878489 45.638489) (width 0.2) (layer "B.Cu") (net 2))
 (segment (start 58.42 42.667) (end 58.42 43.18) (width 0.2) (layer "B.Cu") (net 2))
 (segment (start 58.547 57.536) (end 58.547 53.832) (width 0.25) (layer "F.Cu") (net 14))
 (segment (start 58.547 53.832) (end 57.547 52.832) (width 0.25) (layer "F.Cu") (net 14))
 (segment (start 57.531 50.165) (end 57.531 46.096) (width 0.25) (layer "F.Cu") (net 11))
 (segment (start 57.531 46.096) (end 58.42 45.207) (width 0.25) (layer "F.Cu") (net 11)))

